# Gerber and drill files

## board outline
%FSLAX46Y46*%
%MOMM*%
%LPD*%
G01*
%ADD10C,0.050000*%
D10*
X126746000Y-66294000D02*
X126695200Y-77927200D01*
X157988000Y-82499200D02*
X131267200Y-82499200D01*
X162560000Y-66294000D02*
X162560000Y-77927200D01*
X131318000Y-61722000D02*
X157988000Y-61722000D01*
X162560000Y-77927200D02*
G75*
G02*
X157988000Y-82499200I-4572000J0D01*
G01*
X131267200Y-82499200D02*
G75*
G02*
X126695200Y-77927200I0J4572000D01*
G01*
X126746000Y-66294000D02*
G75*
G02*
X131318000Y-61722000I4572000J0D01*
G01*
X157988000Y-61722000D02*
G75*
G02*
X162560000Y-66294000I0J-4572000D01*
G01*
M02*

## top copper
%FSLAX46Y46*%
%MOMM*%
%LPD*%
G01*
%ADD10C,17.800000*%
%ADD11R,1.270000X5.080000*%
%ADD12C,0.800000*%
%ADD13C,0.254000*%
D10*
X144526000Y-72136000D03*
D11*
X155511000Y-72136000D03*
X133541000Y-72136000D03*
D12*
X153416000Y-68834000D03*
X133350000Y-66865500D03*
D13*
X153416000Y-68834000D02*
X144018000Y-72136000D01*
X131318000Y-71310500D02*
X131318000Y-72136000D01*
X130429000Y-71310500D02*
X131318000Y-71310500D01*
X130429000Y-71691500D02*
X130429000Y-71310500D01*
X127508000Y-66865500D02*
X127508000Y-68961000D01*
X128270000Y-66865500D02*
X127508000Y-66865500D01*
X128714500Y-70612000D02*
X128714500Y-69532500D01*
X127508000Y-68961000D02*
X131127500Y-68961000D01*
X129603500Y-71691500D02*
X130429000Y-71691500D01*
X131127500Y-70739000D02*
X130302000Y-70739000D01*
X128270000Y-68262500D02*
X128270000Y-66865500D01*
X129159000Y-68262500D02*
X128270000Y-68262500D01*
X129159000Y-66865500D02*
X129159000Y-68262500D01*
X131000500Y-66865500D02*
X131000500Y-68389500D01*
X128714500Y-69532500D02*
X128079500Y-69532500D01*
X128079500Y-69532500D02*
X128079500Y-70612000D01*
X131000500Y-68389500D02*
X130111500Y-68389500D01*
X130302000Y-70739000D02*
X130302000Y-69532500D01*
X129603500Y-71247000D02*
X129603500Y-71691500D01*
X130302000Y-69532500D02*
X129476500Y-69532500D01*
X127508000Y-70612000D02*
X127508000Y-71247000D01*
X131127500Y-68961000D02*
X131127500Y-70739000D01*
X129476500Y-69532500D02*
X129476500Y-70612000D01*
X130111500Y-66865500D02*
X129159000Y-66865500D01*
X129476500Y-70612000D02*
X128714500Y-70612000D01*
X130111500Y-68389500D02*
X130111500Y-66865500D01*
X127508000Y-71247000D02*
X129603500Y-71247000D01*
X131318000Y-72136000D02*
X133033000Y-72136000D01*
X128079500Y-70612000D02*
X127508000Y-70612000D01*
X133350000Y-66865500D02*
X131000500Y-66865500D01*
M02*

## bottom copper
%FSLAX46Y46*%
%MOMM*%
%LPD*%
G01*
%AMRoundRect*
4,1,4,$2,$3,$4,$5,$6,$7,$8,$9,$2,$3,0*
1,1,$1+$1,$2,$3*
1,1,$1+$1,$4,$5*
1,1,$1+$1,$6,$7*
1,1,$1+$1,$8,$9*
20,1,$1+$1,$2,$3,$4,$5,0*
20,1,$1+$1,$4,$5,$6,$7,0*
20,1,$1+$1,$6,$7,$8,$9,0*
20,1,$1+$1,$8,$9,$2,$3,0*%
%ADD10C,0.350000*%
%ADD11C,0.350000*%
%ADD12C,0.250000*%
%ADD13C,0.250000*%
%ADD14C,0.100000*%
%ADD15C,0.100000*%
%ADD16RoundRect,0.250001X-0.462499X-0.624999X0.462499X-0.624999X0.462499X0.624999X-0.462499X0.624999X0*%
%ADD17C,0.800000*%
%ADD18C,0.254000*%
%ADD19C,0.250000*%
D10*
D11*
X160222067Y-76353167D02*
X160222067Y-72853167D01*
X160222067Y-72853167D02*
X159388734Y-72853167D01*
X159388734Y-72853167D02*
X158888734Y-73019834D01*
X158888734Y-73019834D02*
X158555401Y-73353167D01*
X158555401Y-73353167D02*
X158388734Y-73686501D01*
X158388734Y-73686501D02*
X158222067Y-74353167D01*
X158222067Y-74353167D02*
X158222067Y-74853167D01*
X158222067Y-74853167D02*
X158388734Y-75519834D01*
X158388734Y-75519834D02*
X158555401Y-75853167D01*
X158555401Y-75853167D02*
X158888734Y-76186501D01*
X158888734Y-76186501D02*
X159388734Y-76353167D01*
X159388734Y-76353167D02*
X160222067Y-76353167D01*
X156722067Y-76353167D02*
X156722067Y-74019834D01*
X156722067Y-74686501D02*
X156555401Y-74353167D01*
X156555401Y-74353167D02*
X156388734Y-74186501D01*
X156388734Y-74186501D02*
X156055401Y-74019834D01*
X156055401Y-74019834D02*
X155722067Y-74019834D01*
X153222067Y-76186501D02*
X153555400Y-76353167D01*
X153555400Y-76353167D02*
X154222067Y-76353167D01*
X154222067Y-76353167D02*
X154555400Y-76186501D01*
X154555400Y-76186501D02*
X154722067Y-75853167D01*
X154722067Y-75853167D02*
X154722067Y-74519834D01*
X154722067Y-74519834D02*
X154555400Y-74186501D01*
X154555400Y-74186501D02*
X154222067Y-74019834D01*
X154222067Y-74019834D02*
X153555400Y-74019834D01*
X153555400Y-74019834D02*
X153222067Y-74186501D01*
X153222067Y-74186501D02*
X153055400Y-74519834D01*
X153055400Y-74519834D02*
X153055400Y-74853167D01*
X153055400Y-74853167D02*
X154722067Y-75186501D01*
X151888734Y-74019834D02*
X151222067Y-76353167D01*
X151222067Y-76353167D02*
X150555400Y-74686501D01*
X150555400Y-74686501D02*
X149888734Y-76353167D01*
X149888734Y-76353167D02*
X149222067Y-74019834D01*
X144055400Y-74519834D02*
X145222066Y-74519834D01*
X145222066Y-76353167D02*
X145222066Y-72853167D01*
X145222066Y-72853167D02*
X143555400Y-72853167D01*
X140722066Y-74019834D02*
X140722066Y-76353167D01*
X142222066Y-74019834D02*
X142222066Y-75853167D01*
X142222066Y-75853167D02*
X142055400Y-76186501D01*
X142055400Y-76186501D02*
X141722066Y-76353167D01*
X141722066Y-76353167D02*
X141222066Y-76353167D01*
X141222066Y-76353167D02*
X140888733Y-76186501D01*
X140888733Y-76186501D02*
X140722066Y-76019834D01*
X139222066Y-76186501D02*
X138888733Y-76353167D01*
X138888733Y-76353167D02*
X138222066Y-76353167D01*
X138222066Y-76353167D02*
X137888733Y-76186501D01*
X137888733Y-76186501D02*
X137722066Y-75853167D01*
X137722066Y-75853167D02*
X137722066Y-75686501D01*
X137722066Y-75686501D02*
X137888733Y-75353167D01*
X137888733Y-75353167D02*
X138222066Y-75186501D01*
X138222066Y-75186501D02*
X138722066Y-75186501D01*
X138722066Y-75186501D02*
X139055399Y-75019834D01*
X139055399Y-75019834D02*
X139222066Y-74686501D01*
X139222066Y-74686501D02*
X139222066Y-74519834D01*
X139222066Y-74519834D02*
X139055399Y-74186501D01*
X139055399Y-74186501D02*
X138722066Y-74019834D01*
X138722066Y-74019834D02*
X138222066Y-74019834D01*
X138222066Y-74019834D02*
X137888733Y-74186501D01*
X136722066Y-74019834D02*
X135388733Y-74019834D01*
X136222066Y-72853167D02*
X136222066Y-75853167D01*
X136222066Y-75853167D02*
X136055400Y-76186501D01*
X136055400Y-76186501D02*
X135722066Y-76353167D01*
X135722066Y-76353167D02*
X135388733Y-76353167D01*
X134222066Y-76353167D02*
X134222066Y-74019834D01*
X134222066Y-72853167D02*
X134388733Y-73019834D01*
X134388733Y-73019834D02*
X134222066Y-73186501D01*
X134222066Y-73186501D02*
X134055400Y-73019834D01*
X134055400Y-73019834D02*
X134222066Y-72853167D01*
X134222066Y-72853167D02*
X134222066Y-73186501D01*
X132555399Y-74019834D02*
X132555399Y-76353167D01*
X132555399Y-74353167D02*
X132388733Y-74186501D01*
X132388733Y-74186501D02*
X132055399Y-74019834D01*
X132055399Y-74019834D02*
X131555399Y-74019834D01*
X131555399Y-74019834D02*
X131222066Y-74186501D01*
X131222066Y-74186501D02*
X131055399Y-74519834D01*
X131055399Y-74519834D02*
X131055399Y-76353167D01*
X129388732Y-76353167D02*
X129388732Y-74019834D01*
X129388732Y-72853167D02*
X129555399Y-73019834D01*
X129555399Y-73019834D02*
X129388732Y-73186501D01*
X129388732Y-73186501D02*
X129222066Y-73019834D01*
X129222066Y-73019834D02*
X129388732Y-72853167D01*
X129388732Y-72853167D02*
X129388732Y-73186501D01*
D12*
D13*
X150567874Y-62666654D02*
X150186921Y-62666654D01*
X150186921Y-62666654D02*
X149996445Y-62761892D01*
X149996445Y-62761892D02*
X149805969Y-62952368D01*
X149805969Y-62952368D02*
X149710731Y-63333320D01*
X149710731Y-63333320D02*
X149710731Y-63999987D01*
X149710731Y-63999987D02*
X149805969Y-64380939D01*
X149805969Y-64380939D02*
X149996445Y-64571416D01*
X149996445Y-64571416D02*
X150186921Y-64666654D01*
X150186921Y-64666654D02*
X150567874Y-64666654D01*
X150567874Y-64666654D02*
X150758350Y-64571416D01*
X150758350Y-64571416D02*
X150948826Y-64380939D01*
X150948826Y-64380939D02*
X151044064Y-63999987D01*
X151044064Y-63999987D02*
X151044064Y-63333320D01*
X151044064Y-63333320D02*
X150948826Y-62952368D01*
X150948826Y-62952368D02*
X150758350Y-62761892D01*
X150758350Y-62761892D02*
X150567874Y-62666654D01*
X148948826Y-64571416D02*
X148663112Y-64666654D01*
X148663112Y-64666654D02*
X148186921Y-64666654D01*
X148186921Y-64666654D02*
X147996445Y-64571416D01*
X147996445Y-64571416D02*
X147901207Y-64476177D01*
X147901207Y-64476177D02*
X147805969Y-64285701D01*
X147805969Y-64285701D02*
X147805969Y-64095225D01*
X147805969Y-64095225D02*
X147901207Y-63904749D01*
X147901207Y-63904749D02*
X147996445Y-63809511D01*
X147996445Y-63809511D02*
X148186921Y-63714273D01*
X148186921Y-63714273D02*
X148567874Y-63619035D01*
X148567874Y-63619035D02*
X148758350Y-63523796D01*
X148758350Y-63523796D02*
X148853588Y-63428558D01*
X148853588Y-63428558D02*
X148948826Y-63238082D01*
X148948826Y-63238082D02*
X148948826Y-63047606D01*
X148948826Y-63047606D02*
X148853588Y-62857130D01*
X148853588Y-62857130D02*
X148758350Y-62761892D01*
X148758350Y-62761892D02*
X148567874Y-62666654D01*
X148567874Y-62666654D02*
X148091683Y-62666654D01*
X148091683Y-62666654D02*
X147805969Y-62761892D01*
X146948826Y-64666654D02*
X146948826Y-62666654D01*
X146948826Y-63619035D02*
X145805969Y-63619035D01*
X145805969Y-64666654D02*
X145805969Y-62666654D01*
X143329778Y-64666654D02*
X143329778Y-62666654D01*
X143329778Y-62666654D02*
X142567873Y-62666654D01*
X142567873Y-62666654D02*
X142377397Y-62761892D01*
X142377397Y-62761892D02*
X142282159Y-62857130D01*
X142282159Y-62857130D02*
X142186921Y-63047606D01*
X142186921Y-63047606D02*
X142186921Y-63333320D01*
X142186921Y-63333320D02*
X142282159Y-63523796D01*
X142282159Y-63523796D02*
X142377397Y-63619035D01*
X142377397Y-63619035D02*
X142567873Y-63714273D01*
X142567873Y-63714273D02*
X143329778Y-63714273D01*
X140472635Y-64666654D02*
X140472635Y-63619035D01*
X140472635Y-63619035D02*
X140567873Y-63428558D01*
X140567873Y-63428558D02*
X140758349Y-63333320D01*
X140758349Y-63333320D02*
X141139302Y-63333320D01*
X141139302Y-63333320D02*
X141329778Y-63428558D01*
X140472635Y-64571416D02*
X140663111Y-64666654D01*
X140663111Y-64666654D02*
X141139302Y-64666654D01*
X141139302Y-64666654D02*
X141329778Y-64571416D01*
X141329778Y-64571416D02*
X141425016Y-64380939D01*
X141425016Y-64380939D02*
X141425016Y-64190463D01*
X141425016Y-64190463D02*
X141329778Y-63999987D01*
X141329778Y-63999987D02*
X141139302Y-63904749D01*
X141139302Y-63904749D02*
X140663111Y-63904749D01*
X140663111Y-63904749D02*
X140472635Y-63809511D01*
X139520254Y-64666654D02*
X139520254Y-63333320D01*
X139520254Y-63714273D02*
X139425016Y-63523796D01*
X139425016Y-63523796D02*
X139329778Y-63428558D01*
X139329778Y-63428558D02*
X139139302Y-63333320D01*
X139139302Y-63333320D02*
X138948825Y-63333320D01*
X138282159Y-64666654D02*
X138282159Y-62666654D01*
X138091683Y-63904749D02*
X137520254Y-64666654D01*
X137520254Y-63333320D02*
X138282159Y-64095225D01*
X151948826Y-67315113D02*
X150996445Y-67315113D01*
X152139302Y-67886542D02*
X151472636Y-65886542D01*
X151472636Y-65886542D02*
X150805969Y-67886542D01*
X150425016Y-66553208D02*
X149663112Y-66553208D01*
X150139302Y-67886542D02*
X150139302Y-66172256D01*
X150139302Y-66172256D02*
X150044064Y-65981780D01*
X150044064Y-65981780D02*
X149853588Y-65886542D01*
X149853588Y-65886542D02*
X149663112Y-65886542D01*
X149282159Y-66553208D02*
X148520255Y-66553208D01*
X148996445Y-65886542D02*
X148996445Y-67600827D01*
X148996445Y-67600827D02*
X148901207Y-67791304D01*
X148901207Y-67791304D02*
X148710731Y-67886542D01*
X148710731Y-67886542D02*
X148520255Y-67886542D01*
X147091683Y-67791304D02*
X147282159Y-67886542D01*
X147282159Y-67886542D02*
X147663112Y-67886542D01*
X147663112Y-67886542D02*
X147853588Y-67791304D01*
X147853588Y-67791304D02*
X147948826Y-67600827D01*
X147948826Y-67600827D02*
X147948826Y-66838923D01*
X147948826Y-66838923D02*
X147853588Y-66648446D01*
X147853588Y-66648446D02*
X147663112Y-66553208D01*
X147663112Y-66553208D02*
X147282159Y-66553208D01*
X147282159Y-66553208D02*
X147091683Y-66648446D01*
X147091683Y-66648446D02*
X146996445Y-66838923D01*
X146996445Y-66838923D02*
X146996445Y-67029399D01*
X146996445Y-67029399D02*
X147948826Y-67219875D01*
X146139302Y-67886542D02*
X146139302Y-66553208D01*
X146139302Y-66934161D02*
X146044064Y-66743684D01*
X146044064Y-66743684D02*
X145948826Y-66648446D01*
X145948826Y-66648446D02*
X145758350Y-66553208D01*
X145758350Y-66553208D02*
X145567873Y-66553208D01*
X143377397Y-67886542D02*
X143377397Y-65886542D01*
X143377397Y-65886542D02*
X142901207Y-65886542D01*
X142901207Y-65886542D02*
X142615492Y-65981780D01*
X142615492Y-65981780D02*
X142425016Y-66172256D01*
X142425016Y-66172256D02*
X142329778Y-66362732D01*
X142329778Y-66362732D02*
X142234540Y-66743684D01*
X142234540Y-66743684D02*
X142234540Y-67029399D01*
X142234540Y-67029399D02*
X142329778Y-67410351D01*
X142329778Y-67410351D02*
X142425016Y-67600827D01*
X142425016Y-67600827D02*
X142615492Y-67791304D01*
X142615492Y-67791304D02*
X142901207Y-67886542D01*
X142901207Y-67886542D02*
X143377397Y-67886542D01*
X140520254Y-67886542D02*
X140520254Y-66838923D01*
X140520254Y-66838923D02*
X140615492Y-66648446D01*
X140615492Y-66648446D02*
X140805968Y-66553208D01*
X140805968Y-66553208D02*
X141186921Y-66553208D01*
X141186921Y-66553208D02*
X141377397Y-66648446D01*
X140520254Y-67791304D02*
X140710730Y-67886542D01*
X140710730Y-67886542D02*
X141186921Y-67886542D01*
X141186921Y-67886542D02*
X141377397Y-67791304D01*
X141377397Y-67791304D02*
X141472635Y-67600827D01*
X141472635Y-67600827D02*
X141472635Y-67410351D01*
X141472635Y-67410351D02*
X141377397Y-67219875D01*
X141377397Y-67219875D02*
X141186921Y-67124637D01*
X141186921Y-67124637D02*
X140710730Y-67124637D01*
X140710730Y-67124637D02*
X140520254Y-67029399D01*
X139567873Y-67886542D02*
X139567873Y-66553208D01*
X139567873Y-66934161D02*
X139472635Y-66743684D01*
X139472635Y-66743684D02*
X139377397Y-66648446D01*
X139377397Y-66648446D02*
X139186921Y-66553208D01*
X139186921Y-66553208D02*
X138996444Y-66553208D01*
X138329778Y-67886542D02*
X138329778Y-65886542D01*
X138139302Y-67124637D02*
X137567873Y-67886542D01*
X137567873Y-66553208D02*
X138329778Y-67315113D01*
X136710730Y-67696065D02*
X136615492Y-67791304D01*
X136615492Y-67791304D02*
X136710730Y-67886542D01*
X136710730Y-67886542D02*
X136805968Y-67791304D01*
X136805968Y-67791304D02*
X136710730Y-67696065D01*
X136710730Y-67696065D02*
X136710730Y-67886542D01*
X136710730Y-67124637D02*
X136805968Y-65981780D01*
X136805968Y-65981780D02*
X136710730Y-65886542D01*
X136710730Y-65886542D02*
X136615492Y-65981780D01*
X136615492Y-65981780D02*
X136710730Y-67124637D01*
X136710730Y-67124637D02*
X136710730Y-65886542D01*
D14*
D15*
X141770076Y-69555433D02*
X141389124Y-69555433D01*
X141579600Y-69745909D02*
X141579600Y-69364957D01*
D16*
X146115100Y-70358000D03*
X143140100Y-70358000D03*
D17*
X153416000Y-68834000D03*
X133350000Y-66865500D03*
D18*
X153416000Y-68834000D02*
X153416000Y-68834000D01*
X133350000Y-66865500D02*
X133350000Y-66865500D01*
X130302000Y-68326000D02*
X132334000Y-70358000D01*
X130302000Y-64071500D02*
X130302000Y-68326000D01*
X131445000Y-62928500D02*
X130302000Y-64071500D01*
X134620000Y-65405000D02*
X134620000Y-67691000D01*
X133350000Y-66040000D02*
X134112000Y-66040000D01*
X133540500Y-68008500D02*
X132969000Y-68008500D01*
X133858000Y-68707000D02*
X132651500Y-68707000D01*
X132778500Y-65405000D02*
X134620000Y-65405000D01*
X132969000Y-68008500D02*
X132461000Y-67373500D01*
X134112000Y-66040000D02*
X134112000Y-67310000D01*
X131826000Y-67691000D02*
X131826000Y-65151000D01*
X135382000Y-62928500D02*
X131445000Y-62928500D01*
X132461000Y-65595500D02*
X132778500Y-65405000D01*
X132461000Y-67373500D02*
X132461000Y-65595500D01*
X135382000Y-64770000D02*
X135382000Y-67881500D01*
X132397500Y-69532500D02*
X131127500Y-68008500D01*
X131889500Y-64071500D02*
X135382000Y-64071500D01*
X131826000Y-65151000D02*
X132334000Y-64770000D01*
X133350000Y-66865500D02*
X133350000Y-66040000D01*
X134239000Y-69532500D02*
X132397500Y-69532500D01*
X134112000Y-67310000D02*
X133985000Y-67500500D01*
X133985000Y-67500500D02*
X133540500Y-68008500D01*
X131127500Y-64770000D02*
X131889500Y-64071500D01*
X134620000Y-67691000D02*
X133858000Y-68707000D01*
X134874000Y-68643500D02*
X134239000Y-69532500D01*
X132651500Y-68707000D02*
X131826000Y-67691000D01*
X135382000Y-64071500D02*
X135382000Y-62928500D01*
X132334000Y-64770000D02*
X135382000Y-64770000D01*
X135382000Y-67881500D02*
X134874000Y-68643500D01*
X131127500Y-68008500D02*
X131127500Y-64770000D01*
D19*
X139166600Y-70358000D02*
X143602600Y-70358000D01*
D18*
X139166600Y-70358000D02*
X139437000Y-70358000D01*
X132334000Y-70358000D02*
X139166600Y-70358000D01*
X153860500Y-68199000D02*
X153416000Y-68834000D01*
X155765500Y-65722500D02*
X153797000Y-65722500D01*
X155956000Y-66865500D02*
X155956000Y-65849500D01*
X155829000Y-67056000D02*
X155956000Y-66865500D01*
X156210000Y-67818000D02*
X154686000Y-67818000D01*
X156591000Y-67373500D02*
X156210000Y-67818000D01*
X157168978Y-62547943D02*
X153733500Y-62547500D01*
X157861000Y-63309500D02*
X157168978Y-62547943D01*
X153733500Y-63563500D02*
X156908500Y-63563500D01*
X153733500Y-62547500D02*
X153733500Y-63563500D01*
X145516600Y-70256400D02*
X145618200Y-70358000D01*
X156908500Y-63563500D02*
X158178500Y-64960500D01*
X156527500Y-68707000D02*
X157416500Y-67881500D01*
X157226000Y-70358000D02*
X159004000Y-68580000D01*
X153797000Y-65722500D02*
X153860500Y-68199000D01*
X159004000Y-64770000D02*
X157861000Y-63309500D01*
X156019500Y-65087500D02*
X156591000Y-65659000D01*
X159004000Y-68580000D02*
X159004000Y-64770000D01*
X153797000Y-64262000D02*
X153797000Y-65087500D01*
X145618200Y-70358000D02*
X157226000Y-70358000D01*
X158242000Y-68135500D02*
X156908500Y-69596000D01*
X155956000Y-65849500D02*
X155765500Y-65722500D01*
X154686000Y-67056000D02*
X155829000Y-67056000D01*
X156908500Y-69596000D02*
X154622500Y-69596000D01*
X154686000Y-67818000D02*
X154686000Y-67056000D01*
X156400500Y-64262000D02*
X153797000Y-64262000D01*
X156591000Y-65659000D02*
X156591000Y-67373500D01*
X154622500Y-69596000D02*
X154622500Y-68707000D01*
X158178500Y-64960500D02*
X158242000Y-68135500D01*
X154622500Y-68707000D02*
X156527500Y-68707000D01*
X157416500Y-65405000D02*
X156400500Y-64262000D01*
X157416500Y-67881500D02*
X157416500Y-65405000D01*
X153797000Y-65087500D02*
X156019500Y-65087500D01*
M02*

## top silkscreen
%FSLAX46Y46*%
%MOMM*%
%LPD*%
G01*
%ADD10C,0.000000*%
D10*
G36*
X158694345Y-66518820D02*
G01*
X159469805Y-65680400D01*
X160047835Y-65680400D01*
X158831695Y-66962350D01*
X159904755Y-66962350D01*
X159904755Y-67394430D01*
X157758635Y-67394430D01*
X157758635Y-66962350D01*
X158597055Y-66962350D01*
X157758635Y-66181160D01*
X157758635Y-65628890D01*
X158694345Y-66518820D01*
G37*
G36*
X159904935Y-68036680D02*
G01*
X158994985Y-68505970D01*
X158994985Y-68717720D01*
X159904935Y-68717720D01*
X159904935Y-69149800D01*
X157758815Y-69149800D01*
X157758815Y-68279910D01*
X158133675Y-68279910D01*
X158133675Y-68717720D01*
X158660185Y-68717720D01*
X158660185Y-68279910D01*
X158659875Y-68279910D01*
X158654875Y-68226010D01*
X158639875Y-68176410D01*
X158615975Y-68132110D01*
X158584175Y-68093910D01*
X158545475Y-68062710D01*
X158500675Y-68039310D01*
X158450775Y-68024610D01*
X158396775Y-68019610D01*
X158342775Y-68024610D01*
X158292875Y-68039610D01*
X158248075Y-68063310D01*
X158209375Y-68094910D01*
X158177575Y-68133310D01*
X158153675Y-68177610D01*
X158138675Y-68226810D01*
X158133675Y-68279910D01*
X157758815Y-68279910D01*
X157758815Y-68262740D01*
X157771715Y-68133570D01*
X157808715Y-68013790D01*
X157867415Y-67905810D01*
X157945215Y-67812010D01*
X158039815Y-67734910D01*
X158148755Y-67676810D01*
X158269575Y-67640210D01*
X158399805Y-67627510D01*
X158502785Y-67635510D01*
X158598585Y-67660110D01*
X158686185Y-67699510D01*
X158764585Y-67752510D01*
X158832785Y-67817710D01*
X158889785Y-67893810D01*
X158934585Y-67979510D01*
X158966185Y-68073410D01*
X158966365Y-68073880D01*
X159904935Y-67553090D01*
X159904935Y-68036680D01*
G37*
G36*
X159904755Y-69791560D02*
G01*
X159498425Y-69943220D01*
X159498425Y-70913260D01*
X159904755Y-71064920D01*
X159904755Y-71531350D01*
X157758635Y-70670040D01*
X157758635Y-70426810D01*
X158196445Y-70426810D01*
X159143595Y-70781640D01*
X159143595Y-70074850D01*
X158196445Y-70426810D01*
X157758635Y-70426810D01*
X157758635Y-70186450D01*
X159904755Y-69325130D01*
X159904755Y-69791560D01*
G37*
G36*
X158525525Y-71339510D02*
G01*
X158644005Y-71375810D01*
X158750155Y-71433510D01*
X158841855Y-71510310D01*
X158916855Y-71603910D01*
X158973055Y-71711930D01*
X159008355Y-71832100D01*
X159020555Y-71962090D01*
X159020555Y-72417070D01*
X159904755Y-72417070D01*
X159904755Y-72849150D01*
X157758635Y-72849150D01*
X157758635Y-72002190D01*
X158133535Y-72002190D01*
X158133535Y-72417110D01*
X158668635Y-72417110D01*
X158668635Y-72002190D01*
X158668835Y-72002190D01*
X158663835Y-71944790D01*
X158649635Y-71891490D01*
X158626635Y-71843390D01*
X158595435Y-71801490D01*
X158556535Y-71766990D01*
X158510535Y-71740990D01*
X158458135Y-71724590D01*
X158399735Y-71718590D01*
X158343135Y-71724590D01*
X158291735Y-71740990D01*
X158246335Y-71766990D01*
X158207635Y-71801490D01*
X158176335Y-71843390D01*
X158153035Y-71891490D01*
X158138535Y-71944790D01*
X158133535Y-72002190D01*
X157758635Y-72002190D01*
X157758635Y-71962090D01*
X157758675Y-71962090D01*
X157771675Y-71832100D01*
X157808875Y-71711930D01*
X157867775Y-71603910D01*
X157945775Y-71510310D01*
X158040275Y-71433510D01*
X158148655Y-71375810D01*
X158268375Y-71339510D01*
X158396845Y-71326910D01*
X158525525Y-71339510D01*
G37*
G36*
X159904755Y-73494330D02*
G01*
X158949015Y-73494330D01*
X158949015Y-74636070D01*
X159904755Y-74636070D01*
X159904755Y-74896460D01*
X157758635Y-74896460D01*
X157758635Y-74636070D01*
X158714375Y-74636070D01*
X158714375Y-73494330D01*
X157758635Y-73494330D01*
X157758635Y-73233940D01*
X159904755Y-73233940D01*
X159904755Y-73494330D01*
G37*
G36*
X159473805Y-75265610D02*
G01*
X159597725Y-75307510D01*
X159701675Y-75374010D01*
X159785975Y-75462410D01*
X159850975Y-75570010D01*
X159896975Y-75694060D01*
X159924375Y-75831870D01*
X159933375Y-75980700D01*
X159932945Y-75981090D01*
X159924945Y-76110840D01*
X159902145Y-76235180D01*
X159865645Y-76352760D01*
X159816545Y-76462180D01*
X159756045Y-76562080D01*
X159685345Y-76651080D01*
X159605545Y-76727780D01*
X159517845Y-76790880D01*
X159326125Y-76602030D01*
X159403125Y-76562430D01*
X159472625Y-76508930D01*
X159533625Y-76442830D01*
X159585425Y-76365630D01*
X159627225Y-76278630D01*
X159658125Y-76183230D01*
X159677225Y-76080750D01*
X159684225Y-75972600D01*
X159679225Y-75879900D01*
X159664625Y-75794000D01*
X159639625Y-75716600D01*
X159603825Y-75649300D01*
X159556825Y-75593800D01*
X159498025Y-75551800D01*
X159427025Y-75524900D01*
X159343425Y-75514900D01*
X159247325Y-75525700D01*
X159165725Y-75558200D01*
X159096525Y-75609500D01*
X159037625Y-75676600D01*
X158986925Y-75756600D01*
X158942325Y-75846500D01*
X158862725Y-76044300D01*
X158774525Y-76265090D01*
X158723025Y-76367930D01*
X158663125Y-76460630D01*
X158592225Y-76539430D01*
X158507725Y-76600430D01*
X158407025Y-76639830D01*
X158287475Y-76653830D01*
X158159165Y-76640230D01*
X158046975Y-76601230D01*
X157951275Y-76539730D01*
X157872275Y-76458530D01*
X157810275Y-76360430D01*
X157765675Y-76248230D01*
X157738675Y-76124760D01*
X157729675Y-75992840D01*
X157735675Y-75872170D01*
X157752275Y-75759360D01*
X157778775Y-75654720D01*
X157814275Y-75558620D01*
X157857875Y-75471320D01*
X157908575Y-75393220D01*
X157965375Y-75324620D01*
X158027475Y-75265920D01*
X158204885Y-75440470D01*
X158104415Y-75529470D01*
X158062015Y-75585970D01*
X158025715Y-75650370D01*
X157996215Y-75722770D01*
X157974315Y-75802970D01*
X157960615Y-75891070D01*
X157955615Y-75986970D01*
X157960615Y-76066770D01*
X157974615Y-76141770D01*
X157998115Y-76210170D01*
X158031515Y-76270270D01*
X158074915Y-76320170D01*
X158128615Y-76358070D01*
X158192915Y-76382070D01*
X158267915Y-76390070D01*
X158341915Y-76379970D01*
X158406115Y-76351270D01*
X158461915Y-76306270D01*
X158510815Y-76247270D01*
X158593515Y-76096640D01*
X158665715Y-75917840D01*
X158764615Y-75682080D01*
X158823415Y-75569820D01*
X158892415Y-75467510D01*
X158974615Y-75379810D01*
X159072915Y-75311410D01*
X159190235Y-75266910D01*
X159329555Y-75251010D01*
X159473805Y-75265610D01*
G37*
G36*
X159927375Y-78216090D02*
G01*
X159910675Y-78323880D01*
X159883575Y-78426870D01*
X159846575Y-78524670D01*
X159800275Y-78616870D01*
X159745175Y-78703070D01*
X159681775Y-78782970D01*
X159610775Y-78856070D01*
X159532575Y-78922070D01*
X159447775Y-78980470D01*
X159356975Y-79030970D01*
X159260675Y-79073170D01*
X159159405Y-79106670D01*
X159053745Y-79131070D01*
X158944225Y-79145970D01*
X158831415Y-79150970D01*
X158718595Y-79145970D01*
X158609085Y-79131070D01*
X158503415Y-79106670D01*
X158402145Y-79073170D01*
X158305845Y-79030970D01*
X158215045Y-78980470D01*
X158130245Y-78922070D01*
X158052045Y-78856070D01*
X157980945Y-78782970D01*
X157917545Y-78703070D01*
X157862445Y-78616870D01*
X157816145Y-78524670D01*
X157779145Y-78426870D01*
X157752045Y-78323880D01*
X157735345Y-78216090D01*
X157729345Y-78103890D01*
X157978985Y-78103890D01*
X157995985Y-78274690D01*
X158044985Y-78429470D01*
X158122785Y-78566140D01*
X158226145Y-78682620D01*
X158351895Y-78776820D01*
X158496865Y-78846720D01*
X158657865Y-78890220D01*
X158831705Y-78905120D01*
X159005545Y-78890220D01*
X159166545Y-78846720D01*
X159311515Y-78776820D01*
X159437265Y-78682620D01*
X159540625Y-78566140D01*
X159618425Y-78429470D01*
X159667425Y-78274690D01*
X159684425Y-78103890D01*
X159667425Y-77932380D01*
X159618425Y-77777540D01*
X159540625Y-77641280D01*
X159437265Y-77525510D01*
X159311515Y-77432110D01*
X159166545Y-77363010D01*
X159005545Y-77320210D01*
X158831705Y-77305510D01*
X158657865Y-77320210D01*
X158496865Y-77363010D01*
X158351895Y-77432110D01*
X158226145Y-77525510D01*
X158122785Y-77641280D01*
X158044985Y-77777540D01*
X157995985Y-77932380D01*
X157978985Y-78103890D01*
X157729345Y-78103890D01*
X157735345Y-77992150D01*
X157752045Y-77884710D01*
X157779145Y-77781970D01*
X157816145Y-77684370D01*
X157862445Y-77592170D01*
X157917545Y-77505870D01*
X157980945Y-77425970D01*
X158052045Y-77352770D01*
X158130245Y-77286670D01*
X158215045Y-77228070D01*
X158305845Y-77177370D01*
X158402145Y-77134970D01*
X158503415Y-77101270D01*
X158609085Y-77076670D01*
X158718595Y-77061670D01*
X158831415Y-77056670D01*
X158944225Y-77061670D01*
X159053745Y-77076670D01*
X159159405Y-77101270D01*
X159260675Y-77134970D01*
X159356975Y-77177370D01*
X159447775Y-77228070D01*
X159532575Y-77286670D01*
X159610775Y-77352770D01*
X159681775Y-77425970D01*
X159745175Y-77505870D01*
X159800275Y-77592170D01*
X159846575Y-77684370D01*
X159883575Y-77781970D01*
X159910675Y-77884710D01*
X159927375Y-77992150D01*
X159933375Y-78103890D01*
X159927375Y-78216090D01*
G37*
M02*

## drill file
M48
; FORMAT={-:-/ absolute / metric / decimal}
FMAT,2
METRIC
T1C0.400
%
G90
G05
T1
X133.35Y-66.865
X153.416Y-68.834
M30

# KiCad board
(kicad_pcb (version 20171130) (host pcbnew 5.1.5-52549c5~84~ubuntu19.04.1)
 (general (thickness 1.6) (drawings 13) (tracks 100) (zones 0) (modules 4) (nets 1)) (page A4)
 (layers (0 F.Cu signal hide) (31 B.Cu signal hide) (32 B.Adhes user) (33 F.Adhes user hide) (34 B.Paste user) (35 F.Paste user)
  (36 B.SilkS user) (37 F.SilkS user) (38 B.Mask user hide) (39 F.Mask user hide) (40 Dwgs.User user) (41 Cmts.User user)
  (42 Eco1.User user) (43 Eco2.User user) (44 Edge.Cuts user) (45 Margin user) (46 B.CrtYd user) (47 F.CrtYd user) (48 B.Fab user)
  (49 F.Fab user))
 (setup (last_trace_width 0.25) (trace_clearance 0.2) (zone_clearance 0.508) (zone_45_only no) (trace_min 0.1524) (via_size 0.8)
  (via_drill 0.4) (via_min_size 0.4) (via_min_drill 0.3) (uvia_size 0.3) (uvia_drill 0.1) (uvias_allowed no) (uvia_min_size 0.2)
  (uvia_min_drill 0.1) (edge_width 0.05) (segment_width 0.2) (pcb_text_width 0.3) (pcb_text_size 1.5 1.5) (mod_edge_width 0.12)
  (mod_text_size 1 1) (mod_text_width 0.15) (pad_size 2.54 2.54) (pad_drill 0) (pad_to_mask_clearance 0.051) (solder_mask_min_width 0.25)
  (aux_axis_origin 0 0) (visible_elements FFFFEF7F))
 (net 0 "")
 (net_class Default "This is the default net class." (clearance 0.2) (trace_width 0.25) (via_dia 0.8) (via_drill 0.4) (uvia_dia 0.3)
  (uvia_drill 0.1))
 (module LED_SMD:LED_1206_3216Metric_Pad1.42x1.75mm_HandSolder (layer B.Cu) (at 144.6276 70.358)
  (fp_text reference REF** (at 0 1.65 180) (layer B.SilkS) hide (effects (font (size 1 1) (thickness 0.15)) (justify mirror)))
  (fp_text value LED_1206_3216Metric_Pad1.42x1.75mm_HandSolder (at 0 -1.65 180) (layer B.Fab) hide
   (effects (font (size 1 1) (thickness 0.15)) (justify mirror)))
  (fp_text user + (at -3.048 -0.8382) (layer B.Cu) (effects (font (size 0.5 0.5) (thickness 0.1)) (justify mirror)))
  (pad 2 smd roundrect (at 1.4875 0) (size 1.425 1.75) (layers B.Cu B.Paste B.Mask) (roundrect_rratio 0.175439))
  (pad 1 smd roundrect (at -1.4875 0) (size 1.425 1.75) (layers B.Cu B.Paste B.Mask) (roundrect_rratio 0.175439)))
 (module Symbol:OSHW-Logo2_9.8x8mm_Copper (layer F.Cu) (at 131.572 79.502)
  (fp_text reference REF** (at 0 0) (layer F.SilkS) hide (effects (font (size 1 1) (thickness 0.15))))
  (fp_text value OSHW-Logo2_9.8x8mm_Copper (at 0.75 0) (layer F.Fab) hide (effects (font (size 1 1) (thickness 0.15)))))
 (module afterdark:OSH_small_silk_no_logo (layer F.Cu) (at 151.638 72.39 90)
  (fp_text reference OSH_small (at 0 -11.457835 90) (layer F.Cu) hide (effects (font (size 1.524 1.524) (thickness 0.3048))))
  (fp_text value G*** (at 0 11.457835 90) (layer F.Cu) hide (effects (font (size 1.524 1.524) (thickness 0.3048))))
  (fp_poly
   (pts (xy 6.76111 6.120635) (xy 6.20884 6.120635) (xy 5.42765 6.959055) (xy 5.42765 6.120635) (xy 4.99557 6.120635) (xy 4.99557 8.266755)
    (xy 5.42765 8.266755) (xy 5.42765 7.193695) (xy 6.7096 8.409835) (xy 6.7096 7.831805) (xy 5.87118 7.056345) (xy 6.76111 6.120635))
   (layer F.SilkS) (width 0))
  (fp_poly
   (pts (xy 4.31659 7.328185) (xy 4.11009 7.022185) (xy 3.67228 7.022185) (xy 3.67228 6.495675) (xy 4.11009 6.495675) (xy 4.16319 6.500675)
    (xy 4.21239 6.515675) (xy 4.25669 6.539575) (xy 4.29509 6.571375) (xy 4.32669 6.610075) (xy 4.35039 6.654875) (xy 4.36539 6.704775)
    (xy 4.37039 6.758775) (xy 4.36539 6.812775) (xy 4.35069 6.862675) (xy 4.32729 6.907475) (xy 4.29609 6.946175) (xy 4.25789 6.977975)
    (xy 4.21359 7.001875) (xy 4.16399 7.016875) (xy 4.11009 7.021875) (xy 4.11009 7.022185) (xy 4.31659 7.328185) (xy 4.41049 7.296585)
    (xy 4.49619 7.251785) (xy 4.57229 7.194785) (xy 4.63749 7.126585) (xy 4.69049 7.048185) (xy 4.72989 6.960585) (xy 4.75449 6.864785)
    (xy 4.76249 6.761805) (xy 4.74979 6.631575) (xy 4.71319 6.510755) (xy 4.65509 6.401815) (xy 4.57799 6.307215) (xy 4.48419 6.229415)
    (xy 4.37621 6.170715) (xy 4.25643 6.133715) (xy 4.12726 6.120815) (xy 3.2402 6.120815) (xy 3.2402 8.266935) (xy 3.67228 8.266935)
    (xy 3.67228 7.356985) (xy 3.88403 7.356985) (xy 4.35332 8.266935) (xy 4.83691 8.266935) (xy 4.31612 7.328365) (xy 4.31659 7.328185))
   (layer F.SilkS) (width 0))
  (fp_poly
   (pts (xy 2.59844 8.266755) (xy 1.96319 6.558445) (xy 2.31515 7.505595) (xy 1.60836 7.505595) (xy 1.96319 6.558445) (xy 2.59844 8.266755)
    (xy 3.06487 8.266755) (xy 2.20355 6.120635) (xy 1.71996 6.120635) (xy 0.85865 8.266755) (xy 1.32508 8.266755) (xy 1.47674 7.860425)
    (xy 2.44678 7.860425) (xy 2.59844 8.266755))
   (layer F.SilkS) (width 0))
  (fp_poly
   (pts (xy 0.42791 6.120635) (xy -0.02711 6.495535) (xy 0.38781 6.495535) (xy 0.44521 6.500535) (xy 0.49851 6.515035) (xy 0.54661 6.538335)
    (xy 0.58851 6.569635) (xy 0.62301 6.608335) (xy 0.64901 6.653735) (xy 0.66541 6.705135) (xy 0.67141 6.761735) (xy 0.66541 6.820135)
    (xy 0.64901 6.872535) (xy 0.62301 6.918535) (xy 0.58851 6.957435) (xy 0.54661 6.988635) (xy 0.49851 7.011635) (xy 0.44521 7.025835)
    (xy 0.38781 7.030835) (xy 0.38781 7.030635) (xy -0.02711 7.030635) (xy -0.02711 6.495535) (xy 0.42791 6.120635) (xy -0.45915 6.120635)
    (xy -0.45915 8.266755) (xy -0.02707 8.266755) (xy -0.02707 7.382555) (xy 0.42791 7.382555) (xy 0.5579 7.370355) (xy 0.67807 7.335055)
    (xy 0.78609 7.278855) (xy 0.87969 7.203855) (xy 0.95649 7.112155) (xy 1.01419 7.006005) (xy 1.05049 6.887525) (xy 1.06309 6.758845)
    (xy 1.05049 6.630375) (xy 1.01419 6.510655) (xy 0.95649 6.402275) (xy 0.87969 6.307775) (xy 0.78609 6.229775) (xy 0.67807 6.170875)
    (xy 0.5579 6.133675) (xy 0.42791 6.120675) (xy 0.42791 6.120635))
   (layer F.SilkS) (width 0))
  (fp_poly
   (pts (xy -1.10433 6.120635) (xy -1.10433 7.076375) (xy -2.24607 7.076375) (xy -2.24607 6.120635) (xy -2.50646 6.120635)
    (xy -2.50646 8.266755) (xy -2.24607 8.266755) (xy -2.24607 7.311015) (xy -1.10433 7.311015) (xy -1.10433 8.266755)
    (xy -0.84394 8.266755) (xy -0.84394 6.120635) (xy -1.10433 6.120635))
   (layer F.SilkS) (width 0))
  (fp_poly
   (pts (xy -3.5907 8.295375) (xy -3.44187 8.286375) (xy -3.30406 8.258975) (xy -3.18001 8.212975) (xy -3.07241 8.147975)
    (xy -2.98401 8.063675) (xy -2.91751 7.959725) (xy -2.87561 7.835805) (xy -2.86101 7.691555) (xy -2.87691 7.552235)
    (xy -2.92141 7.434915) (xy -2.98981 7.336615) (xy -3.07751 7.254415) (xy -3.17982 7.185415) (xy -3.29208 7.126615)
    (xy -3.52784 7.027715) (xy -3.70664 6.955515) (xy -3.85727 6.872815) (xy -3.91627 6.823915) (xy -3.96127 6.768115)
    (xy -3.98997 6.703915) (xy -4.00007 6.629915) (xy -3.99207 6.554915) (xy -3.96807 6.490615) (xy -3.93017 6.436915)
    (xy -3.88027 6.393515) (xy -3.82017 6.360115) (xy -3.75177 6.336615) (xy -3.67677 6.322615) (xy -3.59697 6.317615)
    (xy -3.50107 6.322615) (xy -3.41297 6.336315) (xy -3.33277 6.358215) (xy -3.26037 6.387715) (xy -3.19597 6.424015)
    (xy -3.13947 6.466415) (xy -3.05047 6.566885) (xy -2.87592 6.389475) (xy -2.93462 6.327375) (xy -3.00322 6.270575)
    (xy -3.08132 6.219875) (xy -3.16862 6.176275) (xy -3.26472 6.140775) (xy -3.36936 6.114275) (xy -3.48217 6.097675)
    (xy -3.60284 6.091675) (xy -3.73476 6.100675) (xy -3.85823 6.127675) (xy -3.97043 6.172275) (xy -4.06853 6.234275)
    (xy -4.14973 6.313275) (xy -4.21123 6.408975) (xy -4.25023 6.521165) (xy -4.26383 6.649475) (xy -4.24983 6.769025)
    (xy -4.21043 6.869725) (xy -4.14943 6.954225) (xy -4.07063 7.025125) (xy -3.97793 7.085025) (xy -3.87509 7.136525) (xy -3.6543 7.224725)
    (xy -3.4565 7.304325) (xy -3.3666 7.348925) (xy -3.2866 7.399625) (xy -3.2195 7.458525) (xy -3.1682 7.527725) (xy -3.1357 7.609325)
    (xy -3.1249 7.705425) (xy -3.1349 7.789025) (xy -3.1618 7.860025) (xy -3.2038 7.918825) (xy -3.2593 7.965825) (xy -3.3266 8.001625)
    (xy -3.404 8.026625) (xy -3.4899 8.041225) (xy -3.5826 8.046225) (xy -3.69075 8.039225) (xy -3.79323 8.020125) (xy -3.88863 7.989225)
    (xy -3.97563 7.947425) (xy -4.05283 7.895625) (xy -4.11893 7.834625) (xy -4.17243 7.765125) (xy -4.21203 7.688125)
    (xy -4.40088 7.879845) (xy -4.33778 7.967545) (xy -4.26108 8.047345) (xy -4.17208 8.118045) (xy -4.07218 8.178545)
    (xy -3.96276 8.227645) (xy -3.84518 8.264145) (xy -3.72084 8.286945) (xy -3.59109 8.294945) (xy -3.5907 8.295375))
   (layer F.SilkS) (width 0))
  (fp_poly
   (pts (xy -5.71389 8.295375) (xy -5.71389 8.046425) (xy -5.88469 8.029425) (xy -6.03947 7.980425) (xy -6.17614 7.902625)
    (xy -6.29262 7.799265) (xy -6.38682 7.673515) (xy -6.45672 7.528545) (xy -6.50022 7.367545) (xy -6.51512 7.193705)
    (xy -6.50022 7.019865) (xy -6.45672 6.858865) (xy -6.38682 6.713895) (xy -6.29262 6.588145) (xy -6.17614 6.484785)
    (xy -6.03947 6.406985) (xy -5.88469 6.357985) (xy -5.71389 6.340985) (xy -5.54238 6.357985) (xy -5.38754 6.406985)
    (xy -5.25128 6.484785) (xy -5.13551 6.588145) (xy -5.04211 6.713895) (xy -4.97301 6.858865) (xy -4.93021 7.019865)
    (xy -4.91551 7.193705) (xy -4.93021 7.367545) (xy -4.97301 7.528545) (xy -5.04211 7.673515) (xy -5.13551 7.799265)
    (xy -5.25128 7.902625) (xy -5.38754 7.980425) (xy -5.54238 8.029425) (xy -5.71389 8.046425) (xy -5.71389 8.295375)
    (xy -5.60215 8.289375) (xy -5.49471 8.272675) (xy -5.39197 8.245575) (xy -5.29437 8.208575) (xy -5.20217 8.162275)
    (xy -5.11587 8.107175) (xy -5.03597 8.043775) (xy -4.96277 7.972775) (xy -4.89667 7.894575) (xy -4.83807 7.809775)
    (xy -4.78737 7.718975) (xy -4.74497 7.622675) (xy -4.71127 7.521405) (xy -4.68667 7.415745) (xy -4.67167 7.306225)
    (xy -4.66667 7.193415) (xy -4.67167 7.080595) (xy -4.68667 6.971085) (xy -4.71127 6.865415) (xy -4.74497 6.764145)
    (xy -4.78737 6.667845) (xy -4.83807 6.577045) (xy -4.89667 6.492245) (xy -4.96277 6.414045) (xy -5.03597 6.342945)
    (xy -5.11587 6.279545) (xy -5.20217 6.224445) (xy -5.29437 6.178145) (xy -5.39197 6.141145) (xy -5.49471 6.114045)
    (xy -5.60215 6.097345) (xy -5.71389 6.091345) (xy -5.82609 6.097345) (xy -5.93388 6.114045) (xy -6.03687 6.141145)
    (xy -6.13467 6.178145) (xy -6.22687 6.224445) (xy -6.31307 6.279545) (xy -6.39297 6.342945) (xy -6.46607 6.414045)
    (xy -6.53207 6.492245) (xy -6.59047 6.577045) (xy -6.64097 6.667845) (xy -6.68317 6.764145) (xy -6.71667 6.865415)
    (xy -6.74107 6.971085) (xy -6.75597 7.080595) (xy -6.76097 7.193415) (xy -6.75597 7.306225) (xy -6.74107 7.415745)
    (xy -6.71667 7.521405) (xy -6.68317 7.622675) (xy -6.64097 7.718975) (xy -6.59047 7.809775) (xy -6.53207 7.894575)
    (xy -6.46607 7.972775) (xy -6.39297 8.043775) (xy -6.31307 8.107175) (xy -6.22687 8.162275) (xy -6.13467 8.208575)
    (xy -6.03687 8.245575) (xy -5.93388 8.272675) (xy -5.82609 8.289375) (xy -5.71389 8.295375))
   (layer F.SilkS) (width 0)))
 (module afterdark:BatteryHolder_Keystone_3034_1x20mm (layer F.Cu) (at 144.526 72.136)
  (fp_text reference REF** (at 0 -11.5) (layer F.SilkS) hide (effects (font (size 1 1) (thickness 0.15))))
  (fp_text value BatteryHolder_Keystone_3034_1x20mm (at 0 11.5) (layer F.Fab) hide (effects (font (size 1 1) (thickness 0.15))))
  (pad 2 smd circle (at 0 0) (size 17.8 17.8) (layers F.Cu F.Mask))
  (pad 1 smd rect (at 10.985 0) (size 1.27 5.08) (layers F.Cu F.Paste F.Mask))
  (pad 1 smd rect (at -10.985 0) (size 1.27 5.08) (layers F.Cu F.Paste F.Mask)))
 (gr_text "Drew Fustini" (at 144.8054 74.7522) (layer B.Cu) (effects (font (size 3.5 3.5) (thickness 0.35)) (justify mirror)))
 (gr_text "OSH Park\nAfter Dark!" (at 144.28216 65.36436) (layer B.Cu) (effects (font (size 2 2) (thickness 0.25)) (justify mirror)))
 (gr_line (start 126.746 66.294) (end 126.6952 77.9272) (layer Edge.Cuts) (width 0.05))
 (gr_line (start 157.988 82.4992) (end 131.2672 82.4992) (layer Edge.Cuts) (width 0.05))
 (gr_line (start 162.56 66.294) (end 162.56 77.9272) (layer Edge.Cuts) (width 0.05))
 (gr_line (start 131.318 61.722) (end 157.988 61.722) (layer Edge.Cuts) (width 0.05))
 (gr_arc (start 157.988 77.9272) (end 157.988 82.4992) (angle -90) (layer Edge.Cuts) (width 0.05))
 (gr_arc (start 131.2672 77.9272) (end 126.6952 77.9272) (angle -90) (layer Edge.Cuts) (width 0.05))
 (gr_arc (start 131.318 66.294) (end 131.318 61.722) (angle -90) (layer Edge.Cuts) (width 0.05))
 (gr_arc (start 157.988 66.294) (end 162.56 66.294) (angle -90) (layer Edge.Cuts) (width 0.05))
 (segment (start 153.416 68.834) (end 153.416 68.834) (width 0.254) (layer B.Cu) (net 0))
 (via (at 153.416 68.834) (size 0.8) (drill 0.4) (layers F.Cu B.Cu) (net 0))
 (segment (start 153.416 68.834) (end 144.018 72.136) (width 0.254) (layer F.Cu) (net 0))
 (segment (start 131.318 71.3105) (end 131.318 72.136) (width 0.254) (layer F.Cu) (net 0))
 (segment (start 130.429 71.3105) (end 131.318 71.3105) (width 0.254) (layer F.Cu) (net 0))
 (segment (start 130.429 71.6915) (end 130.429 71.3105) (width 0.254) (layer F.Cu) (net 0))
 (segment (start 127.508 66.8655) (end 127.508 68.961) (width 0.254) (layer F.Cu) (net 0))
 (segment (start 128.27 66.8655) (end 127.508 66.8655) (width 0.254) (layer F.Cu) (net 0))
 (segment (start 128.7145 70.612) (end 128.7145 69.5325) (width 0.254) (layer F.Cu) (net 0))
 (segment (start 127.508 68.961) (end 131.1275 68.961) (width 0.254) (layer F.Cu) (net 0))
 (segment (start 129.6035 71.6915) (end 130.429 71.6915) (width 0.254) (layer F.Cu) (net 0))
 (segment (start 131.1275 70.739) (end 130.302 70.739) (width 0.254) (layer F.Cu) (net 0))
 (segment (start 128.27 68.2625) (end 128.27 66.8655) (width 0.254) (layer F.Cu) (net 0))
 (segment (start 129.159 68.2625) (end 128.27 68.2625) (width 0.254) (layer F.Cu) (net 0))
 (segment (start 129.159 66.8655) (end 129.159 68.2625) (width 0.254) (layer F.Cu) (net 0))
 (segment (start 131.0005 66.8655) (end 131.0005 68.3895) (width 0.254) (layer F.Cu) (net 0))
 (segment (start 128.7145 69.5325) (end 128.0795 69.5325) (width 0.254) (layer F.Cu) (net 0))
 (segment (start 128.0795 69.5325) (end 128.0795 70.612) (width 0.254) (layer F.Cu) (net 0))
 (segment (start 131.0005 68.3895) (end 130.1115 68.3895) (width 0.254) (layer F.Cu) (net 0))
 (segment (start 130.302 70.739) (end 130.302 69.5325) (width 0.254) (layer F.Cu) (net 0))
 (segment (start 129.6035 71.247) (end 129.6035 71.6915) (width 0.254) (layer F.Cu) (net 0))
 (segment (start 130.302 69.5325) (end 129.4765 69.5325) (width 0.254) (layer F.Cu) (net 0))
 (segment (start 127.508 70.612) (end 127.508 71.247) (width 0.254) (layer F.Cu) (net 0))
 (segment (start 131.1275 68.961) (end 131.1275 70.739) (width 0.254) (layer F.Cu) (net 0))
 (segment (start 129.4765 69.5325) (end 129.4765 70.612) (width 0.254) (layer F.Cu) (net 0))
 (segment (start 130.1115 66.8655) (end 129.159 66.8655) (width 0.254) (layer F.Cu) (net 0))
 (segment (start 129.4765 70.612) (end 128.7145 70.612) (width 0.254) (layer F.Cu) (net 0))
 (segment (start 130.1115 68.3895) (end 130.1115 66.8655) (width 0.254) (layer F.Cu) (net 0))
 (segment (start 127.508 71.247) (end 129.6035 71.247) (width 0.254) (layer F.Cu) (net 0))
 (segment (start 131.318 72.136) (end 133.033 72.136) (width 0.254) (layer F.Cu) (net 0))
 (segment (start 128.0795 70.612) (end 127.508 70.612) (width 0.254) (layer F.Cu) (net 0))
 (segment (start 133.35 66.8655) (end 131.0005 66.8655) (width 0.254) (layer F.Cu) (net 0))
 (segment (start 133.35 66.8655) (end 133.35 66.8655) (width 0.254) (layer B.Cu) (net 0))
 (via (at 133.35 66.8655) (size 0.8) (drill 0.4) (layers F.Cu B.Cu) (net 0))
 (segment (start 130.302 68.326) (end 132.334 70.358) (width 0.254) (layer B.Cu) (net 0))
 (segment (start 130.302 64.0715) (end 130.302 68.326) (width 0.254) (layer B.Cu) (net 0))
 (segment (start 131.445 62.9285) (end 130.302 64.0715) (width 0.254) (layer B.Cu) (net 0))
 (segment (start 134.62 65.405) (end 134.62 67.691) (width 0.254) (layer B.Cu) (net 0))
 (segment (start 133.35 66.04) (end 134.112 66.04) (width 0.254) (layer B.Cu) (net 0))
 (segment (start 133.5405 68.0085) (end 132.969 68.0085) (width 0.254) (layer B.Cu) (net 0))
 (segment (start 133.858 68.707) (end 132.6515 68.707) (width 0.254) (layer B.Cu) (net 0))
 (segment (start 132.7785 65.405) (end 134.62 65.405) (width 0.254) (layer B.Cu) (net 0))
 (segment (start 132.969 68.0085) (end 132.461 67.3735) (width 0.254) (layer B.Cu) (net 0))
 (segment (start 134.112 66.04) (end 134.112 67.31) (width 0.254) (layer B.Cu) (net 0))
 (segment (start 131.826 67.691) (end 131.826 65.151) (width 0.254) (layer B.Cu) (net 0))
 (segment (start 135.382 62.9285) (end 131.445 62.9285) (width 0.254) (layer B.Cu) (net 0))
 (segment (start 132.461 65.5955) (end 132.7785 65.405) (width 0.254) (layer B.Cu) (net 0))
 (segment (start 132.461 67.3735) (end 132.461 65.5955) (width 0.254) (layer B.Cu) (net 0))
 (segment (start 135.382 64.77) (end 135.382 67.8815) (width 0.254) (layer B.Cu) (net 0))
 (segment (start 132.3975 69.5325) (end 131.1275 68.0085) (width 0.254) (layer B.Cu) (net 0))
 (segment (start 131.8895 64.0715) (end 135.382 64.0715) (width 0.254) (layer B.Cu) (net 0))
 (segment (start 131.826 65.151) (end 132.334 64.77) (width 0.254) (layer B.Cu) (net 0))
 (segment (start 133.35 66.8655) (end 133.35 66.04) (width 0.254) (layer B.Cu) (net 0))
 (segment (start 134.239 69.5325) (end 132.3975 69.5325) (width 0.254) (layer B.Cu) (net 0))
 (segment (start 134.112 67.31) (end 133.985 67.5005) (width 0.254) (layer B.Cu) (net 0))
 (segment (start 133.985 67.5005) (end 133.5405 68.0085) (width 0.254) (layer B.Cu) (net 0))
 (segment (start 131.1275 64.77) (end 131.8895 64.0715) (width 0.254) (layer B.Cu) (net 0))
 (segment (start 134.62 67.691) (end 133.858 68.707) (width 0.254) (layer B.Cu) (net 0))
 (segment (start 134.874 68.6435) (end 134.239 69.5325) (width 0.254) (layer B.Cu) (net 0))
 (segment (start 132.6515 68.707) (end 131.826 67.691) (width 0.254) (layer B.Cu) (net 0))
 (segment (start 135.382 64.0715) (end 135.382 62.9285) (width 0.254) (layer B.Cu) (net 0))
 (segment (start 132.334 64.77) (end 135.382 64.77) (width 0.254) (layer B.Cu) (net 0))
 (segment (start 135.382 67.8815) (end 134.874 68.6435) (width 0.254) (layer B.Cu) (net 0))
 (segment (start 131.1275 68.0085) (end 131.1275 64.77) (width 0.254) (layer B.Cu) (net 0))
 (segment (start 139.1666 70.358) (end 143.6026 70.358) (width 0.25) (layer B.Cu) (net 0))
 (segment (start 139.1666 70.358) (end 139.437 70.358) (width 0.254) (layer B.Cu) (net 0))
 (segment (start 132.334 70.358) (end 139.1666 70.358) (width 0.254) (layer B.Cu) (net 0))
 (segment (start 153.8605 68.199) (end 153.416 68.834) (width 0.254) (layer B.Cu) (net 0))
 (segment (start 155.7655 65.7225) (end 153.797 65.7225) (width 0.254) (layer B.Cu) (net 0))
 (segment (start 155.956 66.8655) (end 155.956 65.8495) (width 0.254) (layer B.Cu) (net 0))
 (segment (start 155.829 67.056) (end 155.956 66.8655) (width 0.254) (layer B.Cu) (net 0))
 (segment (start 156.21 67.818) (end 154.686 67.818) (width 0.254) (layer B.Cu) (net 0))
 (segment (start 156.591 67.3735) (end 156.21 67.818) (width 0.254) (layer B.Cu) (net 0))
 (segment (start 157.168978 62.547943) (end 153.7335 62.5475) (width 0.254) (layer B.Cu) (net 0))
 (segment (start 157.861 63.3095) (end 157.168978 62.547943) (width 0.254) (layer B.Cu) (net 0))
 (segment (start 153.7335 63.5635) (end 156.9085 63.5635) (width 0.254) (layer B.Cu) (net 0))
 (segment (start 153.7335 62.5475) (end 153.7335 63.5635) (width 0.254) (layer B.Cu) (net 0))
 (segment (start 145.5166 70.2564) (end 145.6182 70.358) (width 0.254) (layer B.Cu) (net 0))
 (segment (start 156.9085 63.5635) (end 158.1785 64.9605) (width 0.254) (layer B.Cu) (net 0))
 (segment (start 156.5275 68.707) (end 157.4165 67.8815) (width 0.254) (layer B.Cu) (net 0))
 (segment (start 157.226 70.358) (end 159.004 68.58) (width 0.254) (layer B.Cu) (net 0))
 (segment (start 153.797 65.7225) (end 153.8605 68.199) (width 0.254) (layer B.Cu) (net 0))
 (segment (start 159.004 64.77) (end 157.861 63.3095) (width 0.254) (layer B.Cu) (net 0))
 (segment (start 156.0195 65.0875) (end 156.591 65.659) (width 0.254) (layer B.Cu) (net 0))
 (segment (start 159.004 68.58) (end 159.004 64.77) (width 0.254) (layer B.Cu) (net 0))
 (segment (start 153.797 64.262) (end 153.797 65.0875) (width 0.254) (layer B.Cu) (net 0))
 (segment (start 145.6182 70.358) (end 157.226 70.358) (width 0.254) (layer B.Cu) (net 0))
 (segment (start 158.242 68.1355) (end 156.9085 69.596) (width 0.254) (layer B.Cu) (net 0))
 (segment (start 155.956 65.8495) (end 155.7655 65.7225) (width 0.254) (layer B.Cu) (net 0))
 (segment (start 154.686 67.056) (end 155.829 67.056) (width 0.254) (layer B.Cu) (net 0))
 (segment (start 156.9085 69.596) (end 154.6225 69.596) (width 0.254) (layer B.Cu) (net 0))
 (segment (start 154.686 67.818) (end 154.686 67.056) (width 0.254) (layer B.Cu) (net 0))
 (segment (start 156.4005 64.262) (end 153.797 64.262) (width 0.254) (layer B.Cu) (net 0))
 (segment (start 156.591 65.659) (end 156.591 67.3735) (width 0.254) (layer B.Cu) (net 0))
 (segment (start 154.6225 69.596) (end 154.6225 68.707) (width 0.254) (layer B.Cu) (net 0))
 (segment (start 158.1785 64.9605) (end 158.242 68.1355) (width 0.254) (layer B.Cu) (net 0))
 (segment (start 154.6225 68.707) (end 156.5275 68.707) (width 0.254) (layer B.Cu) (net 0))
 (segment (start 157.4165 65.405) (end 156.4005 64.262) (width 0.254) (layer B.Cu) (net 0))
 (segment (start 157.4165 67.8815) (end 157.4165 65.405) (width 0.254) (layer B.Cu) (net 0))
 (segment (start 153.797 65.0875) (end 156.0195 65.0875) (width 0.254) (layer B.Cu) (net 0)))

